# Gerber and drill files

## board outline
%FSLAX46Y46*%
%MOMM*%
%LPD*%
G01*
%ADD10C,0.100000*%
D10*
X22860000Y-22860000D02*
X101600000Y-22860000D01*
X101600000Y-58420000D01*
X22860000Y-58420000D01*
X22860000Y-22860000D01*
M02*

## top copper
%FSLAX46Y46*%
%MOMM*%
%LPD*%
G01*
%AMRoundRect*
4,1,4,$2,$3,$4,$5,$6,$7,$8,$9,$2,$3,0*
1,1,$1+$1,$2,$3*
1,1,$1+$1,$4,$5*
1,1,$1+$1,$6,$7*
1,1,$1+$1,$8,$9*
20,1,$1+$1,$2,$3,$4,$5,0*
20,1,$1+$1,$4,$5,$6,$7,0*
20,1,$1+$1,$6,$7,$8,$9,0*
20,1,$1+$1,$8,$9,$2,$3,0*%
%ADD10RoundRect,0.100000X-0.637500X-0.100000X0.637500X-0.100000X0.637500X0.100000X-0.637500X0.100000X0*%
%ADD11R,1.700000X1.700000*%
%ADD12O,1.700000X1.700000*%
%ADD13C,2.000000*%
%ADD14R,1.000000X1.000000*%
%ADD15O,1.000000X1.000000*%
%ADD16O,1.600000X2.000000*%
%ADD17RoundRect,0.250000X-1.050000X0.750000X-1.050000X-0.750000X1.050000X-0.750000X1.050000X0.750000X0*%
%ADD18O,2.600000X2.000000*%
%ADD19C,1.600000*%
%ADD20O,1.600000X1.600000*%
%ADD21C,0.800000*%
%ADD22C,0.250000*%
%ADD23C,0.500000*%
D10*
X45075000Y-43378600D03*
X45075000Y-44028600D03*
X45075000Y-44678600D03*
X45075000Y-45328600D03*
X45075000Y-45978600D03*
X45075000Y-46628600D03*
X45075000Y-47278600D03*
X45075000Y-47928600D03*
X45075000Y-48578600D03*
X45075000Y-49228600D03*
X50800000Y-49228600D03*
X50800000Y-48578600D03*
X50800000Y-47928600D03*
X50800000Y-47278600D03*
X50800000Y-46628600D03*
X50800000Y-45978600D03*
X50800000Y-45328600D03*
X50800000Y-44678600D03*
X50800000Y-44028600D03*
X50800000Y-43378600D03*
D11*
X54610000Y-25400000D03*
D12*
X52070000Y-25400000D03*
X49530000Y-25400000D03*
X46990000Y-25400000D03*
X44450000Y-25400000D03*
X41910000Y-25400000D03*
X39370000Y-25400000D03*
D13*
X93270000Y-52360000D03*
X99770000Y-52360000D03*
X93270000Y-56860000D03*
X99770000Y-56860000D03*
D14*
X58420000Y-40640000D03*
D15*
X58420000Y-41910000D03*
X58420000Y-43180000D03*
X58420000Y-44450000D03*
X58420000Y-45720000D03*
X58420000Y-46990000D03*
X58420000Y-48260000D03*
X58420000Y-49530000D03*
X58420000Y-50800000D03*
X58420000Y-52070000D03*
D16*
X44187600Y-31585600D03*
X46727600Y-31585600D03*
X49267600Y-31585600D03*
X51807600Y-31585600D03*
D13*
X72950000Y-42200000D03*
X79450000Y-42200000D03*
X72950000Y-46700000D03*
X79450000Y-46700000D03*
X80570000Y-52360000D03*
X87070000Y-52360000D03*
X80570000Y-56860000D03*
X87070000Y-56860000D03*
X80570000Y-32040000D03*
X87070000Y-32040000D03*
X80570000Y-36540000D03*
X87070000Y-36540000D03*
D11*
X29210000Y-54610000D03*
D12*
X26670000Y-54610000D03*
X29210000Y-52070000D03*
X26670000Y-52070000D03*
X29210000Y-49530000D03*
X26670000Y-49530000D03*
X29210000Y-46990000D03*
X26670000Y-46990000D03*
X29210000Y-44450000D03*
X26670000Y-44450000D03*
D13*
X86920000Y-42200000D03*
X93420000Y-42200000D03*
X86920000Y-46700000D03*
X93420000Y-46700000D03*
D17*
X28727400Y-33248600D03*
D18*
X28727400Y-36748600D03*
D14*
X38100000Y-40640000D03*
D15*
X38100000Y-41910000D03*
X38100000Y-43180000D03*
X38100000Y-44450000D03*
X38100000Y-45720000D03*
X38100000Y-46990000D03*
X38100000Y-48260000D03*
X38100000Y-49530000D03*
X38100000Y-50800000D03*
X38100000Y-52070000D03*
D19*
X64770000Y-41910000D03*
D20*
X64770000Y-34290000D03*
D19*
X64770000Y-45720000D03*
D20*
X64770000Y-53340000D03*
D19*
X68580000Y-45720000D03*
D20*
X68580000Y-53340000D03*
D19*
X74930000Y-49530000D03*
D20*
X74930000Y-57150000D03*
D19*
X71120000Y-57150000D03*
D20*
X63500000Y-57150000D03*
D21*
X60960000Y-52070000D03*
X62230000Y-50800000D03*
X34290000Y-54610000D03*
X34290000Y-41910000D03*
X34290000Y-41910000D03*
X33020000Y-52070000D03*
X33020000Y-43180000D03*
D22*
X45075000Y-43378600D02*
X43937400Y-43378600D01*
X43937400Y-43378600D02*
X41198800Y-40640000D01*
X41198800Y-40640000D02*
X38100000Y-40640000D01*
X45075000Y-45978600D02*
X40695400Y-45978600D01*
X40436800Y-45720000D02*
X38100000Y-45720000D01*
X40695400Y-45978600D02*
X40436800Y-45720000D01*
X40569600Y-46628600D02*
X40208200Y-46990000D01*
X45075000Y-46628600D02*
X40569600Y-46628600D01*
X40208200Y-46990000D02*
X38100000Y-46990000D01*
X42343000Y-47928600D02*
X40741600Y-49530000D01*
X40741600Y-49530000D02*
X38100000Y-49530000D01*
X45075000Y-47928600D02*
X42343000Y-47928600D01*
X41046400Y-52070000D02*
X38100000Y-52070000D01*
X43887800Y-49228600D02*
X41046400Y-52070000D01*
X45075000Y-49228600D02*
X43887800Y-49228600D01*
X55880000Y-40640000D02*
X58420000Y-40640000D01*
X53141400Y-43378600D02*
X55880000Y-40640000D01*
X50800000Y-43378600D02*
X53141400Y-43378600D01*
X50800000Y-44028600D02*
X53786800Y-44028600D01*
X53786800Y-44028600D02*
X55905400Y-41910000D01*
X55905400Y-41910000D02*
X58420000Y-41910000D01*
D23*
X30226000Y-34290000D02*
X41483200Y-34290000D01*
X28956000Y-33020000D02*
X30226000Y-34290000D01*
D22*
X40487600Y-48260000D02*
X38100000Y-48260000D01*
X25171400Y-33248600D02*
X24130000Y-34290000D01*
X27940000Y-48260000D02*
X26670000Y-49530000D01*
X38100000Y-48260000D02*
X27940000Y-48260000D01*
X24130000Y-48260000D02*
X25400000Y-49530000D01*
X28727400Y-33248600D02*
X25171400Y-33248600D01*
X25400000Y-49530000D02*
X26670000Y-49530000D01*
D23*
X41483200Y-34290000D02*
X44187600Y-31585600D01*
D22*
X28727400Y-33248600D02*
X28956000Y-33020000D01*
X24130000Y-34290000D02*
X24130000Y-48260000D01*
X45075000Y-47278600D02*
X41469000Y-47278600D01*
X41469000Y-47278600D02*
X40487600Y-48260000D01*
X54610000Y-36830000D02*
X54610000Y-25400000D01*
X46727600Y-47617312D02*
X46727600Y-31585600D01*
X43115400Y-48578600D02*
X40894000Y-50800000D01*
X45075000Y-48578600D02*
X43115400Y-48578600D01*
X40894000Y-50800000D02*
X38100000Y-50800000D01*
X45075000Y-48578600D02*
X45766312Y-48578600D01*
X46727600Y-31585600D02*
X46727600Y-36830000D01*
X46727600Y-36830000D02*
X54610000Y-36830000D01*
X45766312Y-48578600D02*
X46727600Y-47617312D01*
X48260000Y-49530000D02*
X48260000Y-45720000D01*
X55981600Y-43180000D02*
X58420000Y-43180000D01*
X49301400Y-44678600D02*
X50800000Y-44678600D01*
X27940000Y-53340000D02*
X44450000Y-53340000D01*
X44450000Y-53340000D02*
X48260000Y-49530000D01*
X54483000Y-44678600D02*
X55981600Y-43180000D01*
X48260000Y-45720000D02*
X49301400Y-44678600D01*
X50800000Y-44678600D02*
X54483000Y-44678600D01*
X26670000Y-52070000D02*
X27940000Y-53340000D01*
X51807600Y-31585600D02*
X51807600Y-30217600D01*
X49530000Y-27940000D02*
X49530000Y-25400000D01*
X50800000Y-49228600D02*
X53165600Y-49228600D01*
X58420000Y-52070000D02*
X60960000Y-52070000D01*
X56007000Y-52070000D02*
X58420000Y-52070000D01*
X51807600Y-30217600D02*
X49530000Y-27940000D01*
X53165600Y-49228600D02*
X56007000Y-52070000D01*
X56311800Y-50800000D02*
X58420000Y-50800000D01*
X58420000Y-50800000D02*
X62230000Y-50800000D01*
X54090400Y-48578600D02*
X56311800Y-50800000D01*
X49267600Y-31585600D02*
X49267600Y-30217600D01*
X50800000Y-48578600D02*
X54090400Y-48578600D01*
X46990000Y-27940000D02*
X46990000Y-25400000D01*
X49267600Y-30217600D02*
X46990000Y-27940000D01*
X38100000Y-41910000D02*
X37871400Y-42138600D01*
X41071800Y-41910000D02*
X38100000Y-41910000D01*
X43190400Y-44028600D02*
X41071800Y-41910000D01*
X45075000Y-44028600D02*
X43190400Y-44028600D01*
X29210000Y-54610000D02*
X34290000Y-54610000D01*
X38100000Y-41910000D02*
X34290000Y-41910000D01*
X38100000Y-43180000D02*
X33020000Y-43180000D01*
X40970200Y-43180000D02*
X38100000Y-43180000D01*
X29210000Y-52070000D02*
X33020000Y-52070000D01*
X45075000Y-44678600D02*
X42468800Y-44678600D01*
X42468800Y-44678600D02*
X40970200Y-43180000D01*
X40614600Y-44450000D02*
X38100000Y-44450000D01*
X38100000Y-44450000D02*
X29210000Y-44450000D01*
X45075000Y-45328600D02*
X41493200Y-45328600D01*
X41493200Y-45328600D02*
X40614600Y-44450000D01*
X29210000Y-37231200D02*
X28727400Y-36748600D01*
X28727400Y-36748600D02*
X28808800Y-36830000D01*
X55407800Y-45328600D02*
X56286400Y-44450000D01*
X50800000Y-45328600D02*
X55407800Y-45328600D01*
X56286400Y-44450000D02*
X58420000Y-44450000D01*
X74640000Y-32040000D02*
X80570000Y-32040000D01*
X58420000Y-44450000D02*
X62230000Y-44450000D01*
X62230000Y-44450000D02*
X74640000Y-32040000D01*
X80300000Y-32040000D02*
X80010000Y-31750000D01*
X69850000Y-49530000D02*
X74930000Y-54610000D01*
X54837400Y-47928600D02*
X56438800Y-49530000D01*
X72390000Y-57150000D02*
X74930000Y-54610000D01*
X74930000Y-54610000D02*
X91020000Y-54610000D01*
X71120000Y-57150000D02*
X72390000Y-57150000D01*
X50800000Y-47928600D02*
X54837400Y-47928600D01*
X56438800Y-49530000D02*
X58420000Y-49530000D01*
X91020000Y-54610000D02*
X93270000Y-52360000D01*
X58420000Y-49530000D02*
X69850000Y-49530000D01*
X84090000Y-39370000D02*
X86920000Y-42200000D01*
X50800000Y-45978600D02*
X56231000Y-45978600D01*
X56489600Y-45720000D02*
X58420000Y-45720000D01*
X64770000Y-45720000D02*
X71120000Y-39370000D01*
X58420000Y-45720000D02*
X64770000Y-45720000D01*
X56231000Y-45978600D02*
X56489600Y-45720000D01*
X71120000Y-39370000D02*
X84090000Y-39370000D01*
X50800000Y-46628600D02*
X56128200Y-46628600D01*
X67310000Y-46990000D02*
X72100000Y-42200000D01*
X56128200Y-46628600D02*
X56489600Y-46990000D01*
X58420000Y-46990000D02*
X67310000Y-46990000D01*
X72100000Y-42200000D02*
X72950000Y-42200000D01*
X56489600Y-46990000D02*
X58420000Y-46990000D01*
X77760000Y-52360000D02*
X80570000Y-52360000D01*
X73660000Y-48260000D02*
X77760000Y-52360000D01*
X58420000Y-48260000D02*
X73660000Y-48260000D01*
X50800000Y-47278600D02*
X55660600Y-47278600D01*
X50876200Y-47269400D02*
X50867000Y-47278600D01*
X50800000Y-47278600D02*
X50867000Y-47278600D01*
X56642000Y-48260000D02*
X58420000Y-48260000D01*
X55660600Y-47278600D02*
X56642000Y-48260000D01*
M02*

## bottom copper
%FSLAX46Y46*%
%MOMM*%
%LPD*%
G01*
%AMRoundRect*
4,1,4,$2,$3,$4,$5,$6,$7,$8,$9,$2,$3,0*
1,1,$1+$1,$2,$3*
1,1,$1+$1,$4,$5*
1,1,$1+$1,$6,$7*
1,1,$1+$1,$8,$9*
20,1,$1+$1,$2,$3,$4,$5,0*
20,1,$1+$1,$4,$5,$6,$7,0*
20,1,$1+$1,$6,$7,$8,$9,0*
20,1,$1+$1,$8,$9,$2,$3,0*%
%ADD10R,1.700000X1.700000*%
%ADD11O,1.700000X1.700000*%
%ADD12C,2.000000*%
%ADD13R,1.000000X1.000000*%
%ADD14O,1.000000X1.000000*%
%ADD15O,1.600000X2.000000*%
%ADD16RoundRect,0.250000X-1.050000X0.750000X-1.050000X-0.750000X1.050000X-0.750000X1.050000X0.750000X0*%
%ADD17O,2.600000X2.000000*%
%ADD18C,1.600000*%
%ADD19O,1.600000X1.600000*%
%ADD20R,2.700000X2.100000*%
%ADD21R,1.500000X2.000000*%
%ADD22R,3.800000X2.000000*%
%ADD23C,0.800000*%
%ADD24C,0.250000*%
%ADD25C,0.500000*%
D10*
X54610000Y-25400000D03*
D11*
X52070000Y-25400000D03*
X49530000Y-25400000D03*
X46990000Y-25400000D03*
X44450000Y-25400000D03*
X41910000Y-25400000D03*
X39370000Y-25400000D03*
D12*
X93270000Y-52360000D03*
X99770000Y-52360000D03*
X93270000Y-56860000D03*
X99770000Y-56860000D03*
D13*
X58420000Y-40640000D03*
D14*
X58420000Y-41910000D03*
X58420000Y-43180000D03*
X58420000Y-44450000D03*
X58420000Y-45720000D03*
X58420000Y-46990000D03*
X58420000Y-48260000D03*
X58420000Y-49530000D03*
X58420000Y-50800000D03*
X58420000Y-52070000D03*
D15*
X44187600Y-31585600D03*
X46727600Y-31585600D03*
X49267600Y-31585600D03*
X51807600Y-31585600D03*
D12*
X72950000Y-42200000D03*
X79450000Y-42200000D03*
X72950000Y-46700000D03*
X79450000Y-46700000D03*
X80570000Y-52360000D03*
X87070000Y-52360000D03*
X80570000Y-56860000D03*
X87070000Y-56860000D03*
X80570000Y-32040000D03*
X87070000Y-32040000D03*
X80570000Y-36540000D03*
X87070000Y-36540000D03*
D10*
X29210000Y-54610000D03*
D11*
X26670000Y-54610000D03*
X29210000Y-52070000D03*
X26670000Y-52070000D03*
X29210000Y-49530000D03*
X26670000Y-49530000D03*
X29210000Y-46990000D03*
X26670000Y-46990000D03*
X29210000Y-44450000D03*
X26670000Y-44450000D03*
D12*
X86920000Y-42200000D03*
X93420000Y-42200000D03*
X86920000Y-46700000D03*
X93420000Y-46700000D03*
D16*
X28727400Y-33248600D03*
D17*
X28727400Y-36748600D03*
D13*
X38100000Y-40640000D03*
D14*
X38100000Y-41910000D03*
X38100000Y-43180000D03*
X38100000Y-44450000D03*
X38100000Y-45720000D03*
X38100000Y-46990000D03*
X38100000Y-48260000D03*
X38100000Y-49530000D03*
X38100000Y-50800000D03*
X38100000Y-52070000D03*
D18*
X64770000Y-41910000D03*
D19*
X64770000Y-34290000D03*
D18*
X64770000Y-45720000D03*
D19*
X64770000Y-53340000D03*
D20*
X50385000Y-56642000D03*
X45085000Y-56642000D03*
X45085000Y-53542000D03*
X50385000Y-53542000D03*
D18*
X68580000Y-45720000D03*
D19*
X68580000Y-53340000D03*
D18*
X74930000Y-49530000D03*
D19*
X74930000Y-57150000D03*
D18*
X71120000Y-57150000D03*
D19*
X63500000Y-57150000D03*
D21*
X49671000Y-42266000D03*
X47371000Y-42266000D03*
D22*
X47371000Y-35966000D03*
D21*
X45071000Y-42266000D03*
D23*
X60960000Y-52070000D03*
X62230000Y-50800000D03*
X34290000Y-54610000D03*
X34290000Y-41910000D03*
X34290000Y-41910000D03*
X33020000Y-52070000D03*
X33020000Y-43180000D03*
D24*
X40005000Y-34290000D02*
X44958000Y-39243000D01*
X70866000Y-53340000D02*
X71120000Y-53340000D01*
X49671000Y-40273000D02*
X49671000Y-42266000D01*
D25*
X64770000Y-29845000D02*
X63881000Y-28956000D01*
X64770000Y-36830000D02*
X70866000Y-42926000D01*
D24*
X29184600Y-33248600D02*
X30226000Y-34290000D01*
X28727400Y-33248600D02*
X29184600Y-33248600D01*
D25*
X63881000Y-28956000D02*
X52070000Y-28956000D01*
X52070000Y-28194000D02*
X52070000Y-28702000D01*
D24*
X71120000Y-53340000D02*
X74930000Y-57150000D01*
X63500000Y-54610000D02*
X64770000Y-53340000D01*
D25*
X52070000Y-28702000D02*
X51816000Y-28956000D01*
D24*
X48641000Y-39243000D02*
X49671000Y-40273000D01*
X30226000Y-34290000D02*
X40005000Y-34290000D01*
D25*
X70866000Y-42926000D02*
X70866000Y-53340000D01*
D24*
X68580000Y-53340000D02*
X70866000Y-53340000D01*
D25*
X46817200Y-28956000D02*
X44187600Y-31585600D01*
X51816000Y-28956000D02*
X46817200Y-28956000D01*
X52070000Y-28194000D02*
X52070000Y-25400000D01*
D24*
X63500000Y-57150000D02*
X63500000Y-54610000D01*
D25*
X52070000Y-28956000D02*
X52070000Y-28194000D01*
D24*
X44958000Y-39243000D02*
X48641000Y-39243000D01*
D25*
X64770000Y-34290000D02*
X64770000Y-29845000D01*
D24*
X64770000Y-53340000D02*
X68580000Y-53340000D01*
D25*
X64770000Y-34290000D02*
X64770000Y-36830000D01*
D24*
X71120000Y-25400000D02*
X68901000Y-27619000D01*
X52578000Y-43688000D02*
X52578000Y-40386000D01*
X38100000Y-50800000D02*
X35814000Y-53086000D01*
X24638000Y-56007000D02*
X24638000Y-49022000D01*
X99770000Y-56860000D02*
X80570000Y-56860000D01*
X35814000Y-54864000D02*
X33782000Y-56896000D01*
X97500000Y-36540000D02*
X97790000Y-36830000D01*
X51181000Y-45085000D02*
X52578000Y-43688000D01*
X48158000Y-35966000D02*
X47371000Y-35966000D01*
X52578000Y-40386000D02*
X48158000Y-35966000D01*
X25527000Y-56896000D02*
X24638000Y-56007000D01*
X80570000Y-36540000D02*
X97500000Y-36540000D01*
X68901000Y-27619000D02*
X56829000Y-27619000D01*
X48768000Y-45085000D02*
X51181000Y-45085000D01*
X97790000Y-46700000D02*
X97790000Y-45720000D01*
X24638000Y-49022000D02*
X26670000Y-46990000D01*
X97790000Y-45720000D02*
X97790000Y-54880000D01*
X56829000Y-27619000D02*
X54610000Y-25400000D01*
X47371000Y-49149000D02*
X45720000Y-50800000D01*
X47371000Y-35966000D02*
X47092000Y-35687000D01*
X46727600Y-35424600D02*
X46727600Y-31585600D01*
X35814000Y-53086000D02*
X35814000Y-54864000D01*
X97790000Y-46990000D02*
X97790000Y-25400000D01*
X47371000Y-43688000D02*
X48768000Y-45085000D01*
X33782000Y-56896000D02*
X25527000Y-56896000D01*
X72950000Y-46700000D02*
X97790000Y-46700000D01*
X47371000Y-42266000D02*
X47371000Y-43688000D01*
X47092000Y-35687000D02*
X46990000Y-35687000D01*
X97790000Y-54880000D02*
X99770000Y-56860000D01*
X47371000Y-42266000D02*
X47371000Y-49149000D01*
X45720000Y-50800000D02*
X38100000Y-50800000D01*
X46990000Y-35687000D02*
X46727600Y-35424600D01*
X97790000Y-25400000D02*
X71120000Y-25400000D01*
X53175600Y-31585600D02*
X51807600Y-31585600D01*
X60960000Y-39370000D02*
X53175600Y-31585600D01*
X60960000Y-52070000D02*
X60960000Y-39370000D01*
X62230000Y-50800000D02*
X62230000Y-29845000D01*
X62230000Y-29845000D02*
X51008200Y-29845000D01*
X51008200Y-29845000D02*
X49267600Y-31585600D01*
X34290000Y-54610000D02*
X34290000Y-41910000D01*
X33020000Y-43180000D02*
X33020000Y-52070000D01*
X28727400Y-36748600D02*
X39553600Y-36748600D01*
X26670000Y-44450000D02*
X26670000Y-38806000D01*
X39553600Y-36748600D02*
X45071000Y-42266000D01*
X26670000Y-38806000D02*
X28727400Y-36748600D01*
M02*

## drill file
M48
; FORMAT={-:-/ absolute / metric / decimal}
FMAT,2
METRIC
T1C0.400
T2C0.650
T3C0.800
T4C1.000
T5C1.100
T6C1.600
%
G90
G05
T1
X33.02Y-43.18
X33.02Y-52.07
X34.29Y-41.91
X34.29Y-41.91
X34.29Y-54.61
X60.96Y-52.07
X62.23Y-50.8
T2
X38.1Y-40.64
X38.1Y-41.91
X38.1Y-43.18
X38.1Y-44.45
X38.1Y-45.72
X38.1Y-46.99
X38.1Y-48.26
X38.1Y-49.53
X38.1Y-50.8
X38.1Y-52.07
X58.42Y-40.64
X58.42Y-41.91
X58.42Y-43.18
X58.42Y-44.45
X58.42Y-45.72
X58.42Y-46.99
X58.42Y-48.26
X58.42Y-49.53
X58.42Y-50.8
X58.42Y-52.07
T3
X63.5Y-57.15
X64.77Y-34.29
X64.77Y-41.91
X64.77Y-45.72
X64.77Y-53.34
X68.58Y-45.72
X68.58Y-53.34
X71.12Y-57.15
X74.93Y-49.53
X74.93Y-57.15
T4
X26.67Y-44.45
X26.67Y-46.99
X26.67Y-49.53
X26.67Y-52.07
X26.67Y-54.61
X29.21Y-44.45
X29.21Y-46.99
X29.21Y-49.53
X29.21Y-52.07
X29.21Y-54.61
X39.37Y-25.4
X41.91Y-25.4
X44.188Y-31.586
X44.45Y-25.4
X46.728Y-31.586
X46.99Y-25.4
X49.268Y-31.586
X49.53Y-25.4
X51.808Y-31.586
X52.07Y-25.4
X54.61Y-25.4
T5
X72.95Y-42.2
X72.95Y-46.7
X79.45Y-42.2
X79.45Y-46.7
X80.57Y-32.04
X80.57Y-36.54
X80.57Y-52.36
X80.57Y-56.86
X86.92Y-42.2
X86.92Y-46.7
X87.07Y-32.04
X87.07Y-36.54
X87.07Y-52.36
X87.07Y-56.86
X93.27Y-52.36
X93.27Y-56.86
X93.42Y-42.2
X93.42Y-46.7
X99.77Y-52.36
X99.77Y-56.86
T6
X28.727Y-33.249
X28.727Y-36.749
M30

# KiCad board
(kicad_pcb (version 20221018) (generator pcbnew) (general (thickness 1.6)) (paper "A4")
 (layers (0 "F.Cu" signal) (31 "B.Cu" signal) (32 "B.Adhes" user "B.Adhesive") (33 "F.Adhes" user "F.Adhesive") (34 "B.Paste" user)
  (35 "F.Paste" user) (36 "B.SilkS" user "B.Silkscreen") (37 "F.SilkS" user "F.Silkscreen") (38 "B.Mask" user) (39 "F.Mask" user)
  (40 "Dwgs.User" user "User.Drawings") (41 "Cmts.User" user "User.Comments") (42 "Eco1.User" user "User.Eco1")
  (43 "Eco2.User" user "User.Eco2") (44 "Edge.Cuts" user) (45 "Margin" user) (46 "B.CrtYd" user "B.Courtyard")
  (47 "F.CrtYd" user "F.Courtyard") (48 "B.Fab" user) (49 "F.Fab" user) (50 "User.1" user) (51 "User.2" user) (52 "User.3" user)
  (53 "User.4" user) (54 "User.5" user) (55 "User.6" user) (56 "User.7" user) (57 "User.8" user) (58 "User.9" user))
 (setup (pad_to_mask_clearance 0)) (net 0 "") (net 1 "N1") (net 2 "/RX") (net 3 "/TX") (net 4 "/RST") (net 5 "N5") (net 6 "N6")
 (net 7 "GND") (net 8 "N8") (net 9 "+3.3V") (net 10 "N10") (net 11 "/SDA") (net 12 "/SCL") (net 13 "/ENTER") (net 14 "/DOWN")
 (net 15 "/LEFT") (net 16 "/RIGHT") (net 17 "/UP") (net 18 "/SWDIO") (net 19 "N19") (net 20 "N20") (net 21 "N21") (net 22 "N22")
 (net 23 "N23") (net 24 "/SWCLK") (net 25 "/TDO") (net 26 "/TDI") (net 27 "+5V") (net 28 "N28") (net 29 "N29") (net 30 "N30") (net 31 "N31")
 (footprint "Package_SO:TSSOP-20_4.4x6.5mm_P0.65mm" (layer "F.Cu") (at 47.9375 46.3036)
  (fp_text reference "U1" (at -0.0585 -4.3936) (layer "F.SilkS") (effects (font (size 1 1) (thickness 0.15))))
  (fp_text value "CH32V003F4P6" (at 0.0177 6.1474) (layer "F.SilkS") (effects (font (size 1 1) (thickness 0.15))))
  (pad "1" smd roundrect (at -2.8625 -2.925) (size 1.475 0.4) (layers "F.Cu" "F.Paste" "F.Mask") (roundrect_rratio 0.25) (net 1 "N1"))
  (pad "2" smd roundrect (at -2.8625 -2.275) (size 1.475 0.4) (layers "F.Cu" "F.Paste" "F.Mask") (roundrect_rratio 0.25) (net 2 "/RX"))
  (pad "3" smd roundrect (at -2.8625 -1.625) (size 1.475 0.4) (layers "F.Cu" "F.Paste" "F.Mask") (roundrect_rratio 0.25) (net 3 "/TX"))
  (pad "4" smd roundrect (at -2.8625 -0.975) (size 1.475 0.4) (layers "F.Cu" "F.Paste" "F.Mask") (roundrect_rratio 0.25) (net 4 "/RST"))
  (pad "5" smd roundrect (at -2.8625 -0.325) (size 1.475 0.4) (layers "F.Cu" "F.Paste" "F.Mask") (roundrect_rratio 0.25) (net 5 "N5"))
  (pad "6" smd roundrect (at -2.8625 0.325) (size 1.475 0.4) (layers "F.Cu" "F.Paste" "F.Mask") (roundrect_rratio 0.25) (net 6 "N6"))
  (pad "7" smd roundrect (at -2.8625 0.975) (size 1.475 0.4) (layers "F.Cu" "F.Paste" "F.Mask") (roundrect_rratio 0.25) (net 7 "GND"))
  (pad "8" smd roundrect (at -2.8625 1.625) (size 1.475 0.4) (layers "F.Cu" "F.Paste" "F.Mask") (roundrect_rratio 0.25) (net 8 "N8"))
  (pad "9" smd roundrect (at -2.8625 2.275) (size 1.475 0.4) (layers "F.Cu" "F.Paste" "F.Mask") (roundrect_rratio 0.25) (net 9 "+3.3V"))
  (pad "10" smd roundrect (at -2.8625 2.925) (size 1.475 0.4) (layers "F.Cu" "F.Paste" "F.Mask") (roundrect_rratio 0.25) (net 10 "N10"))
  (pad "11" smd roundrect (at 2.8625 2.925) (size 1.475 0.4) (layers "F.Cu" "F.Paste" "F.Mask") (roundrect_rratio 0.25) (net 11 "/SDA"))
  (pad "12" smd roundrect (at 2.8625 2.275) (size 1.475 0.4) (layers "F.Cu" "F.Paste" "F.Mask") (roundrect_rratio 0.25) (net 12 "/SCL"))
  (pad "13" smd roundrect (at 2.8625 1.625) (size 1.475 0.4) (layers "F.Cu" "F.Paste" "F.Mask") (roundrect_rratio 0.25) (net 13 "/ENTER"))
  (pad "14" smd roundrect (at 2.8625 0.975) (size 1.475 0.4) (layers "F.Cu" "F.Paste" "F.Mask") (roundrect_rratio 0.25) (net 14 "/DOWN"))
  (pad "15" smd roundrect (at 2.8625 0.325) (size 1.475 0.4) (layers "F.Cu" "F.Paste" "F.Mask") (roundrect_rratio 0.25) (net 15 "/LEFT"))
  (pad "16" smd roundrect (at 2.8625 -0.325) (size 1.475 0.4) (layers "F.Cu" "F.Paste" "F.Mask") (roundrect_rratio 0.25) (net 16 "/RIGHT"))
  (pad "17" smd roundrect (at 2.8625 -0.975) (size 1.475 0.4) (layers "F.Cu" "F.Paste" "F.Mask") (roundrect_rratio 0.25) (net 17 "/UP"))
  (pad "18" smd roundrect (at 2.8625 -1.625) (size 1.475 0.4) (layers "F.Cu" "F.Paste" "F.Mask") (roundrect_rratio 0.25) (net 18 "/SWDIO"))
  (pad "19" smd roundrect (at 2.8625 -2.275) (size 1.475 0.4) (layers "F.Cu" "F.Paste" "F.Mask") (roundrect_rratio 0.25) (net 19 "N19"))
  (pad "20" smd roundrect (at 2.8625 -2.925) (size 1.475 0.4) (layers "F.Cu" "F.Paste" "F.Mask") (roundrect_rratio 0.25) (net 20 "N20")))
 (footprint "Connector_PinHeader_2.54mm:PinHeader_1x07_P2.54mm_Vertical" (layer "F.Cu") (at 54.61 25.4 -90)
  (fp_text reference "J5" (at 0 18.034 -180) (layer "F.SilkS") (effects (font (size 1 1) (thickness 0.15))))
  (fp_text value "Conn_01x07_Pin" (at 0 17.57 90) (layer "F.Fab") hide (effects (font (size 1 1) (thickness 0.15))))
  (pad "1" thru_hole rect (at 0 0 270) (size 1.7 1.7) (drill 1) (layers "*.Cu" "*.Mask") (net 9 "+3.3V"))
  (pad "2" thru_hole oval (at 0 2.54 270) (size 1.7 1.7) (drill 1) (layers "*.Cu" "*.Mask") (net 7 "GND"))
  (pad "3" thru_hole oval (at 0 5.08 270) (size 1.7 1.7) (drill 1) (layers "*.Cu" "*.Mask") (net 11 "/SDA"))
  (pad "4" thru_hole oval (at 0 7.62 270) (size 1.7 1.7) (drill 1) (layers "*.Cu" "*.Mask") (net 12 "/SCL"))
  (pad "5" thru_hole oval (at 0 10.16 270) (size 1.7 1.7) (drill 1) (layers "*.Cu" "*.Mask") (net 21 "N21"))
  (pad "6" thru_hole oval (at 0 12.7 270) (size 1.7 1.7) (drill 1) (layers "*.Cu" "*.Mask") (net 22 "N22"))
  (pad "7" thru_hole oval (at 0 15.24 270) (size 1.7 1.7) (drill 1) (layers "*.Cu" "*.Mask") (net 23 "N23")))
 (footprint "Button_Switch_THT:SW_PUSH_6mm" (layer "F.Cu") (at 93.27 52.36)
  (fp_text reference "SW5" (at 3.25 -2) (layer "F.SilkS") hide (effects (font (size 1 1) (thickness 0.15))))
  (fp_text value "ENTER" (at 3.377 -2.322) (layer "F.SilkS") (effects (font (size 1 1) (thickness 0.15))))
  (pad "1" thru_hole circle (at 0 0 90) (size 2 2) (drill 1.1) (layers "*.Cu" "*.Mask") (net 13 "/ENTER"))
  (pad "1" thru_hole circle (at 6.5 0 90) (size 2 2) (drill 1.1) (layers "*.Cu" "*.Mask") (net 13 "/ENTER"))
  (pad "2" thru_hole circle (at 0 4.5 90) (size 2 2) (drill 1.1) (layers "*.Cu" "*.Mask") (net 9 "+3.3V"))
  (pad "2" thru_hole circle (at 6.5 4.5 90) (size 2 2) (drill 1.1) (layers "*.Cu" "*.Mask") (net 9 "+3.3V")))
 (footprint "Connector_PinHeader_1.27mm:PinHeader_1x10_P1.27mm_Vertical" (layer "F.Cu") (at 58.42 40.64)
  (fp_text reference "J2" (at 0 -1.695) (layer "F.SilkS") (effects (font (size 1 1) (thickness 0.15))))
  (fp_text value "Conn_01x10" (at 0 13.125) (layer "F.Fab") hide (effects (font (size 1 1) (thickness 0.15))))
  (pad "1" thru_hole rect (at 0 0) (size 1 1) (drill 0.65) (layers "*.Cu" "*.Mask") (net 20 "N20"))
  (pad "2" thru_hole oval (at 0 1.27) (size 1 1) (drill 0.65) (layers "*.Cu" "*.Mask") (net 19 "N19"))
  (pad "3" thru_hole oval (at 0 2.54) (size 1 1) (drill 0.65) (layers "*.Cu" "*.Mask") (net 18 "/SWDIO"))
  (pad "4" thru_hole oval (at 0 3.81) (size 1 1) (drill 0.65) (layers "*.Cu" "*.Mask") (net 17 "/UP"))
  (pad "5" thru_hole oval (at 0 5.08) (size 1 1) (drill 0.65) (layers "*.Cu" "*.Mask") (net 16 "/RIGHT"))
  (pad "6" thru_hole oval (at 0 6.35) (size 1 1) (drill 0.65) (layers "*.Cu" "*.Mask") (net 15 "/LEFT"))
  (pad "7" thru_hole oval (at 0 7.62) (size 1 1) (drill 0.65) (layers "*.Cu" "*.Mask") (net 14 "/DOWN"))
  (pad "8" thru_hole oval (at 0 8.89) (size 1 1) (drill 0.65) (layers "*.Cu" "*.Mask") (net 13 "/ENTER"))
  (pad "9" thru_hole oval (at 0 10.16) (size 1 1) (drill 0.65) (layers "*.Cu" "*.Mask") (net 12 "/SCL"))
  (pad "10" thru_hole oval (at 0 11.43) (size 1 1) (drill 0.65) (layers "*.Cu" "*.Mask") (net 11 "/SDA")))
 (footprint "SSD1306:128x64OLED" (layer "F.Cu") (at 47.8076 42.1856)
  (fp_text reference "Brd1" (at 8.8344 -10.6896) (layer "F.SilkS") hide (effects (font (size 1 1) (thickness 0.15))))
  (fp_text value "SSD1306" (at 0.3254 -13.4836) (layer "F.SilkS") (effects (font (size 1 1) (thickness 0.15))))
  (pad "1" thru_hole oval (at -3.62 -10.6 90) (size 2 1.6) (drill 1) (layers "*.Cu" "*.Mask") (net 7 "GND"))
  (pad "2" thru_hole oval (at -1.08 -10.6 90) (size 2 1.6) (drill 1) (layers "*.Cu" "*.Mask") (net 9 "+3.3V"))
  (pad "3" thru_hole oval (at 1.46 -10.6 90) (size 2 1.6) (drill 1) (layers "*.Cu" "*.Mask") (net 12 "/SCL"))
  (pad "4" thru_hole oval (at 4 -10.6 90) (size 2 1.6) (drill 1) (layers "*.Cu" "*.Mask") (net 11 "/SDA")))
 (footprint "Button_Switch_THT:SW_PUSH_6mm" (layer "F.Cu") (at 72.95 42.2)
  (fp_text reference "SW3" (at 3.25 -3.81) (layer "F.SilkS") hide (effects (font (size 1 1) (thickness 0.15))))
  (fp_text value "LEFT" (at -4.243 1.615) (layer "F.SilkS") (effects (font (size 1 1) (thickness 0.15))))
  (pad "1" thru_hole circle (at 0 0 90) (size 2 2) (drill 1.1) (layers "*.Cu" "*.Mask") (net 15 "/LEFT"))
  (pad "1" thru_hole circle (at 6.5 0 90) (size 2 2) (drill 1.1) (layers "*.Cu" "*.Mask") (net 15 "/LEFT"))
  (pad "2" thru_hole circle (at 0 4.5 90) (size 2 2) (drill 1.1) (layers "*.Cu" "*.Mask") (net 9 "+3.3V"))
  (pad "2" thru_hole circle (at 6.5 4.5 90) (size 2 2) (drill 1.1) (layers "*.Cu" "*.Mask") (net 9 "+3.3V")))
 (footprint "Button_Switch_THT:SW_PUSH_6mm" (layer "F.Cu") (at 80.57 52.36)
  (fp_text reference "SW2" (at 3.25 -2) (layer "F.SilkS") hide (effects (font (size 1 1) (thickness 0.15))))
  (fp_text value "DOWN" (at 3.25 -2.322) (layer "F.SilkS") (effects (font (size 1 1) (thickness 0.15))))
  (pad "1" thru_hole circle (at 0 0 90) (size 2 2) (drill 1.1) (layers "*.Cu" "*.Mask") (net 14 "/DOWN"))
  (pad "1" thru_hole circle (at 6.5 0 90) (size 2 2) (drill 1.1) (layers "*.Cu" "*.Mask") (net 14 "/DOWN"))
  (pad "2" thru_hole circle (at 0 4.5 90) (size 2 2) (drill 1.1) (layers "*.Cu" "*.Mask") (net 9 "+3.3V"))
  (pad "2" thru_hole circle (at 6.5 4.5 90) (size 2 2) (drill 1.1) (layers "*.Cu" "*.Mask") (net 9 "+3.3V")))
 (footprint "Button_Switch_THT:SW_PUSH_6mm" (layer "F.Cu") (at 80.57 32.04)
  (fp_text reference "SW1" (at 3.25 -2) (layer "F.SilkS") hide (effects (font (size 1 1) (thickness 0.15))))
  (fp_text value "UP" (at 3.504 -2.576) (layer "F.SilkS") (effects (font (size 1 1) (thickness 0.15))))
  (pad "1" thru_hole circle (at 0 0 90) (size 2 2) (drill 1.1) (layers "*.Cu" "*.Mask") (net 17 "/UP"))
  (pad "1" thru_hole circle (at 6.5 0 90) (size 2 2) (drill 1.1) (layers "*.Cu" "*.Mask") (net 17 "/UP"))
  (pad "2" thru_hole circle (at 0 4.5 90) (size 2 2) (drill 1.1) (layers "*.Cu" "*.Mask") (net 9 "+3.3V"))
  (pad "2" thru_hole circle (at 6.5 4.5 90) (size 2 2) (drill 1.1) (layers "*.Cu" "*.Mask") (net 9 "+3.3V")))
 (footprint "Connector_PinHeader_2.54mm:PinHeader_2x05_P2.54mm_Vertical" (layer "F.Cu") (at 29.21 54.61 180)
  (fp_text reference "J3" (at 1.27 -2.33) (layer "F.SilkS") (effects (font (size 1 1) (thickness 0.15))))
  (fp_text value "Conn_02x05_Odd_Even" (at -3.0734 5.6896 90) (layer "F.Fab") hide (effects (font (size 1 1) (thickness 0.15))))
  (pad "1" thru_hole rect (at 0 0 180) (size 1.7 1.7) (drill 1) (layers "*.Cu" "*.Mask") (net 2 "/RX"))
  (pad "2" thru_hole oval (at 2.54 0 180) (size 1.7 1.7) (drill 1) (layers "*.Cu" "*.Mask") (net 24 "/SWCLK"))
  (pad "3" thru_hole oval (at 0 2.54 180) (size 1.7 1.7) (drill 1) (layers "*.Cu" "*.Mask") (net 3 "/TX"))
  (pad "4" thru_hole oval (at 2.54 2.54 180) (size 1.7 1.7) (drill 1) (layers "*.Cu" "*.Mask") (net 18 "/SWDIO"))
  (pad "5" thru_hole oval (at 0 5.08 180) (size 1.7 1.7) (drill 1) (layers "*.Cu" "*.Mask") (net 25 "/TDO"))
  (pad "6" thru_hole oval (at 2.54 5.08 180) (size 1.7 1.7) (drill 1) (layers "*.Cu" "*.Mask") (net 7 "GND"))
  (pad "7" thru_hole oval (at 0 7.62 180) (size 1.7 1.7) (drill 1) (layers "*.Cu" "*.Mask") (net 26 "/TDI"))
  (pad "8" thru_hole oval (at 2.54 7.62 180) (size 1.7 1.7) (drill 1) (layers "*.Cu" "*.Mask") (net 9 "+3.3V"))
  (pad "9" thru_hole oval (at 0 10.16 180) (size 1.7 1.7) (drill 1) (layers "*.Cu" "*.Mask") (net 4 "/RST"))
  (pad "10" thru_hole oval (at 2.54 10.16 180) (size 1.7 1.7) (drill 1) (layers "*.Cu" "*.Mask") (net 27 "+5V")))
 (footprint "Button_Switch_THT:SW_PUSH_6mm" (layer "F.Cu") (at 86.92 42.2)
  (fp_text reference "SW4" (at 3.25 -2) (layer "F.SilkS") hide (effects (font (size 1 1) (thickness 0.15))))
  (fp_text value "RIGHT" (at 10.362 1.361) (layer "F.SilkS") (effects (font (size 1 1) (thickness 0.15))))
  (pad "1" thru_hole circle (at 0 0 90) (size 2 2) (drill 1.1) (layers "*.Cu" "*.Mask") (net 16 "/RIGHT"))
  (pad "1" thru_hole circle (at 6.5 0 90) (size 2 2) (drill 1.1) (layers "*.Cu" "*.Mask") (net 16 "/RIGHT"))
  (pad "2" thru_hole circle (at 0 4.5 90) (size 2 2) (drill 1.1) (layers "*.Cu" "*.Mask") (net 9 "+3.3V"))
  (pad "2" thru_hole circle (at 6.5 4.5 90) (size 2 2) (drill 1.1) (layers "*.Cu" "*.Mask") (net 9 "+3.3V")))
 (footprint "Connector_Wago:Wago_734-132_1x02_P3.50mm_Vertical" (layer "F.Cu") (at 28.7274 33.2486 -90)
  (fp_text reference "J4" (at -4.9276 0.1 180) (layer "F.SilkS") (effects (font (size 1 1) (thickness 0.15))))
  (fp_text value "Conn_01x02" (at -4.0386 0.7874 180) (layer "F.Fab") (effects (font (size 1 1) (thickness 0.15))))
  (pad "1" thru_hole roundrect (at 0 0 270) (size 2 2.6) (drill 1.6) (layers "*.Cu" "*.Mask") (roundrect_rratio 0.125) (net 7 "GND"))
  (pad "2" thru_hole oval (at 3.5 0 270) (size 2 2.6) (drill 1.6) (layers "*.Cu" "*.Mask") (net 27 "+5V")))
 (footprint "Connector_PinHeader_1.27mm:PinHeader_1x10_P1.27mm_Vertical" (layer "F.Cu") (at 38.1 40.64)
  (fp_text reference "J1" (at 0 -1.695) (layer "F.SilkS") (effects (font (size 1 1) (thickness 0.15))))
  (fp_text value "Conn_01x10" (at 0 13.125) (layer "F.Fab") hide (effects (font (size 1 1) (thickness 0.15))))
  (pad "1" thru_hole rect (at 0 0) (size 1 1) (drill 0.65) (layers "*.Cu" "*.Mask") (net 1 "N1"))
  (pad "2" thru_hole oval (at 0 1.27) (size 1 1) (drill 0.65) (layers "*.Cu" "*.Mask") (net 2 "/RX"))
  (pad "3" thru_hole oval (at 0 2.54) (size 1 1) (drill 0.65) (layers "*.Cu" "*.Mask") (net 3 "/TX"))
  (pad "4" thru_hole oval (at 0 3.81) (size 1 1) (drill 0.65) (layers "*.Cu" "*.Mask") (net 4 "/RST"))
  (pad "5" thru_hole oval (at 0 5.08) (size 1 1) (drill 0.65) (layers "*.Cu" "*.Mask") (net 5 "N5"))
  (pad "6" thru_hole oval (at 0 6.35) (size 1 1) (drill 0.65) (layers "*.Cu" "*.Mask") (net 6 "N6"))
  (pad "7" thru_hole oval (at 0 7.62) (size 1 1) (drill 0.65) (layers "*.Cu" "*.Mask") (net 7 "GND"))
  (pad "8" thru_hole oval (at 0 8.89) (size 1 1) (drill 0.65) (layers "*.Cu" "*.Mask") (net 8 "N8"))
  (pad "9" thru_hole oval (at 0 10.16) (size 1 1) (drill 0.65) (layers "*.Cu" "*.Mask") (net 9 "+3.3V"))
  (pad "10" thru_hole oval (at 0 11.43) (size 1 1) (drill 0.65) (layers "*.Cu" "*.Mask") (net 10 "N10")))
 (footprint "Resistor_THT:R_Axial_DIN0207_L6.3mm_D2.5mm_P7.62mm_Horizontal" (layer "B.Cu") (at 64.77 41.91 90)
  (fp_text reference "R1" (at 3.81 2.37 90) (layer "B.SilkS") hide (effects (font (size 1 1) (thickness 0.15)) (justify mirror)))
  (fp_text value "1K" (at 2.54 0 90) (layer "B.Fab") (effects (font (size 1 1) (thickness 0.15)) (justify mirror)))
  (pad "1" thru_hole circle (at 0 0 90) (size 1.6 1.6) (drill 0.8) (layers "*.Cu" "*.Mask") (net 17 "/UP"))
  (pad "2" thru_hole oval (at 7.62 0 90) (size 1.6 1.6) (drill 0.8) (layers "*.Cu" "*.Mask") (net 7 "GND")))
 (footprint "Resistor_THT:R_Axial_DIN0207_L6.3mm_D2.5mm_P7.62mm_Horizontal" (layer "B.Cu") (at 64.77 45.72 -90)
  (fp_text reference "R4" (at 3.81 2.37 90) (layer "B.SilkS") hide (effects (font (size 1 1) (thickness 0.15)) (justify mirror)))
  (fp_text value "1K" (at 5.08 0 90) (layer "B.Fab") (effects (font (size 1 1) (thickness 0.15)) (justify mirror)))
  (pad "1" thru_hole circle (at 0 0 270) (size 1.6 1.6) (drill 0.8) (layers "*.Cu" "*.Mask") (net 16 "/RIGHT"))
  (pad "2" thru_hole oval (at 7.62 0 270) (size 1.6 1.6) (drill 0.8) (layers "*.Cu" "*.Mask") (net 7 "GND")))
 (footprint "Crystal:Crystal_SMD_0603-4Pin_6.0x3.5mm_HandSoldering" (layer "B.Cu") (at 47.735 55.092 180)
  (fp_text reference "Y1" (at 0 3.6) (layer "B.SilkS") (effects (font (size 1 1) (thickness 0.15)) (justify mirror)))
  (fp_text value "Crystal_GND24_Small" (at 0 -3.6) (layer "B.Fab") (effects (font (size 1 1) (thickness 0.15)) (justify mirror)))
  (pad "1" smd rect (at -2.65 -1.55 180) (size 2.7 2.1) (layers "B.Cu" "B.Paste" "B.Mask") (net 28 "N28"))
  (pad "2" smd rect (at 2.65 -1.55 180) (size 2.7 2.1) (layers "B.Cu" "B.Paste" "B.Mask") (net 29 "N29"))
  (pad "3" smd rect (at 2.65 1.55 180) (size 2.7 2.1) (layers "B.Cu" "B.Paste" "B.Mask") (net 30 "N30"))
  (pad "4" smd rect (at -2.65 1.55 180) (size 2.7 2.1) (layers "B.Cu" "B.Paste" "B.Mask") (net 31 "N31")))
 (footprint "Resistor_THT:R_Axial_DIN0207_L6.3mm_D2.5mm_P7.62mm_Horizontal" (layer "B.Cu") (at 68.58 45.72 -90)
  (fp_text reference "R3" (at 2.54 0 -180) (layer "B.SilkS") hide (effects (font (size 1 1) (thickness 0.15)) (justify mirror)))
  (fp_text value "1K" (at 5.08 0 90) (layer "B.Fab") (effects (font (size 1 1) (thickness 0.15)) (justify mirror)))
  (pad "1" thru_hole circle (at 0 0 270) (size 1.6 1.6) (drill 0.8) (layers "*.Cu" "*.Mask") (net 15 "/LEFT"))
  (pad "2" thru_hole oval (at 7.62 0 270) (size 1.6 1.6) (drill 0.8) (layers "*.Cu" "*.Mask") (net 7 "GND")))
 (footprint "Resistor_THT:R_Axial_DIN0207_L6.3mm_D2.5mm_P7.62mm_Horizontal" (layer "B.Cu") (at 74.93 49.53 -90)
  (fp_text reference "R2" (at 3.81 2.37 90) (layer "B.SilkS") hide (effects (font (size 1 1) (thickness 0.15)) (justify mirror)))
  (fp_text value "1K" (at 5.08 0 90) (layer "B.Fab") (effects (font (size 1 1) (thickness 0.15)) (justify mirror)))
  (pad "1" thru_hole circle (at 0 0 270) (size 1.6 1.6) (drill 0.8) (layers "*.Cu" "*.Mask") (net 14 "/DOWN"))
  (pad "2" thru_hole oval (at 7.62 0 270) (size 1.6 1.6) (drill 0.8) (layers "*.Cu" "*.Mask") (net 7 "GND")))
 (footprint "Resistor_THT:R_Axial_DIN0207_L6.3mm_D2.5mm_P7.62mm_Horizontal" (layer "B.Cu") (at 71.12 57.15 180)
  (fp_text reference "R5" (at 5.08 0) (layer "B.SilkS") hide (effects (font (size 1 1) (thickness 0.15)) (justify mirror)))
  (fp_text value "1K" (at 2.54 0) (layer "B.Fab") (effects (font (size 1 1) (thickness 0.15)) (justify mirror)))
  (pad "1" thru_hole circle (at 0 0 180) (size 1.6 1.6) (drill 0.8) (layers "*.Cu" "*.Mask") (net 13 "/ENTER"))
  (pad "2" thru_hole oval (at 7.62 0 180) (size 1.6 1.6) (drill 0.8) (layers "*.Cu" "*.Mask") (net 7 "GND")))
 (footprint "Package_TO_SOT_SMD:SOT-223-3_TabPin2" (layer "B.Cu") (at 47.371 39.116 90)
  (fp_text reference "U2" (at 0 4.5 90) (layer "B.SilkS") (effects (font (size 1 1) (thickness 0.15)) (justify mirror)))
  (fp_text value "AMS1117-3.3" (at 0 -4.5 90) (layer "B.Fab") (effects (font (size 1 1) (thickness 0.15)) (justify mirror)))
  (pad "1" smd rect (at -3.15 2.3 90) (size 2 1.5) (layers "B.Cu" "B.Paste" "B.Mask") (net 7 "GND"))
  (pad "2" smd rect (at -3.15 0 90) (size 2 1.5) (layers "B.Cu" "B.Paste" "B.Mask") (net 9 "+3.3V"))
  (pad "2" smd rect (at 3.15 0 90) (size 2 3.8) (layers "B.Cu" "B.Paste" "B.Mask") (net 9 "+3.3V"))
  (pad "3" smd rect (at -3.15 -2.3 90) (size 2 1.5) (layers "B.Cu" "B.Paste" "B.Mask") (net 27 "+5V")))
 (gr_rect (start 22.86 22.86) (end 101.6 58.42) (stroke (width 0.1) (type default)) (fill none) (layer "Edge.Cuts"))
 (segment (start 45.075 43.3786) (end 43.9374 43.3786) (width 0.25) (layer "F.Cu") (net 1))
 (segment (start 43.9374 43.3786) (end 41.1988 40.64) (width 0.25) (layer "F.Cu") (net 1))
 (segment (start 41.1988 40.64) (end 38.1 40.64) (width 0.25) (layer "F.Cu") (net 1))
 (segment (start 45.075 45.9786) (end 40.6954 45.9786) (width 0.25) (layer "F.Cu") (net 5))
 (segment (start 40.4368 45.72) (end 38.1 45.72) (width 0.25) (layer "F.Cu") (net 5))
 (segment (start 40.6954 45.9786) (end 40.4368 45.72) (width 0.25) (layer "F.Cu") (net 5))
 (segment (start 40.5696 46.6286) (end 40.2082 46.99) (width 0.25) (layer "F.Cu") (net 6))
 (segment (start 45.075 46.6286) (end 40.5696 46.6286) (width 0.25) (layer "F.Cu") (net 6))
 (segment (start 40.2082 46.99) (end 38.1 46.99) (width 0.25) (layer "F.Cu") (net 6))
 (segment (start 42.343 47.9286) (end 40.7416 49.53) (width 0.25) (layer "F.Cu") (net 8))
 (segment (start 40.7416 49.53) (end 38.1 49.53) (width 0.25) (layer "F.Cu") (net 8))
 (segment (start 45.075 47.9286) (end 42.343 47.9286) (width 0.25) (layer "F.Cu") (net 8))
 (segment (start 41.0464 52.07) (end 38.1 52.07) (width 0.25) (layer "F.Cu") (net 10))
 (segment (start 43.8878 49.2286) (end 41.0464 52.07) (width 0.25) (layer "F.Cu") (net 10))
 (segment (start 45.075 49.2286) (end 43.8878 49.2286) (width 0.25) (layer "F.Cu") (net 10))
 (segment (start 55.88 40.64) (end 58.42 40.64) (width 0.25) (layer "F.Cu") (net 20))
 (segment (start 53.1414 43.3786) (end 55.88 40.64) (width 0.25) (layer "F.Cu") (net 20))
 (segment (start 50.8 43.3786) (end 53.1414 43.3786) (width 0.25) (layer "F.Cu") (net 20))
 (segment (start 50.8 44.0286) (end 53.7868 44.0286) (width 0.25) (layer "F.Cu") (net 19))
 (segment (start 53.7868 44.0286) (end 55.9054 41.91) (width 0.25) (layer "F.Cu") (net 19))
 (segment (start 55.9054 41.91) (end 58.42 41.91) (width 0.25) (layer "F.Cu") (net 19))
 (segment (start 30.226 34.29) (end 41.4832 34.29) (width 0.5) (layer "F.Cu") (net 7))
 (segment (start 28.956 33.02) (end 30.226 34.29) (width 0.5) (layer "F.Cu") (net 7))
 (segment (start 40.4876 48.26) (end 38.1 48.26) (width 0.25) (layer "F.Cu") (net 7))
 (segment (start 25.1714 33.2486) (end 24.13 34.29) (width 0.25) (layer "F.Cu") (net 7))
 (segment (start 27.94 48.26) (end 26.67 49.53) (width 0.25) (layer "F.Cu") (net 7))
 (segment (start 38.1 48.26) (end 27.94 48.26) (width 0.25) (layer "F.Cu") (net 7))
 (segment (start 24.13 48.26) (end 25.4 49.53) (width 0.25) (layer "F.Cu") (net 7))
 (segment (start 28.7274 33.2486) (end 25.1714 33.2486) (width 0.25) (layer "F.Cu") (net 7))
 (segment (start 25.4 49.53) (end 26.67 49.53) (width 0.25) (layer "F.Cu") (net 7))
 (segment (start 41.4832 34.29) (end 44.1876 31.5856) (width 0.5) (layer "F.Cu") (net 7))
 (segment (start 28.7274 33.2486) (end 28.956 33.02) (width 0.25) (layer "F.Cu") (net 7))
 (segment (start 24.13 34.29) (end 24.13 48.26) (width 0.25) (layer "F.Cu") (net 7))
 (segment (start 45.075 47.2786) (end 41.469 47.2786) (width 0.25) (layer "F.Cu") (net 7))
 (segment (start 41.469 47.2786) (end 40.4876 48.26) (width 0.25) (layer "F.Cu") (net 7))
 (segment (start 40.005 34.29) (end 44.958 39.243) (width 0.25) (layer "B.Cu") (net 7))
 (segment (start 70.866 53.34) (end 71.12 53.34) (width 0.25) (layer "B.Cu") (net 7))
 (segment (start 49.671 40.273) (end 49.671 42.266) (width 0.25) (layer "B.Cu") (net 7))
 (segment (start 64.77 29.845) (end 63.881 28.956) (width 0.5) (layer "B.Cu") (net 7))
 (segment (start 64.77 36.83) (end 70.866 42.926) (width 0.5) (layer "B.Cu") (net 7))
 (segment (start 29.1846 33.2486) (end 30.226 34.29) (width 0.25) (layer "B.Cu") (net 7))
 (segment (start 28.7274 33.2486) (end 29.1846 33.2486) (width 0.25) (layer "B.Cu") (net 7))
 (segment (start 63.881 28.956) (end 52.07 28.956) (width 0.5) (layer "B.Cu") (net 7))
 (segment (start 52.07 28.194) (end 52.07 28.702) (width 0.5) (layer "B.Cu") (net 7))
 (segment (start 71.12 53.34) (end 74.93 57.15) (width 0.25) (layer "B.Cu") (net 7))
 (segment (start 63.5 54.61) (end 64.77 53.34) (width 0.25) (layer "B.Cu") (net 7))
 (segment (start 52.07 28.702) (end 51.816 28.956) (width 0.5) (layer "B.Cu") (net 7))
 (segment (start 48.641 39.243) (end 49.671 40.273) (width 0.25) (layer "B.Cu") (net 7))
 (segment (start 30.226 34.29) (end 40.005 34.29) (width 0.25) (layer "B.Cu") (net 7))
 (segment (start 70.866 42.926) (end 70.866 53.34) (width 0.5) (layer "B.Cu") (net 7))
 (segment (start 68.58 53.34) (end 70.866 53.34) (width 0.25) (layer "B.Cu") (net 7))
 (segment (start 46.8172 28.956) (end 44.1876 31.5856) (width 0.5) (layer "B.Cu") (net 7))
 (segment (start 51.816 28.956) (end 46.8172 28.956) (width 0.5) (layer "B.Cu") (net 7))
 (segment (start 52.07 28.194) (end 52.07 25.4) (width 0.5) (layer "B.Cu") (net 7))
 (segment (start 63.5 57.15) (end 63.5 54.61) (width 0.25) (layer "B.Cu") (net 7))
 (segment (start 52.07 28.956) (end 52.07 28.194) (width 0.5) (layer "B.Cu") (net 7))
 (segment (start 44.958 39.243) (end 48.641 39.243) (width 0.25) (layer "B.Cu") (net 7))
 (segment (start 64.77 34.29) (end 64.77 29.845) (width 0.5) (layer "B.Cu") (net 7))
 (segment (start 64.77 53.34) (end 68.58 53.34) (width 0.25) (layer "B.Cu") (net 7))
 (segment (start 64.77 34.29) (end 64.77 36.83) (width 0.5) (layer "B.Cu") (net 7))
 (segment (start 54.61 36.83) (end 54.61 25.4) (width 0.25) (layer "F.Cu") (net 9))
 (segment (start 46.7276 47.617312) (end 46.7276 31.5856) (width 0.25) (layer "F.Cu") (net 9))
 (segment (start 43.1154 48.5786) (end 40.894 50.8) (width 0.25) (layer "F.Cu") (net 9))
 (segment (start 45.075 48.5786) (end 43.1154 48.5786) (width 0.25) (layer "F.Cu") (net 9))
 (segment (start 40.894 50.8) (end 38.1 50.8) (width 0.25) (layer "F.Cu") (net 9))
 (segment (start 45.075 48.5786) (end 45.766312 48.5786) (width 0.25) (layer "F.Cu") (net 9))
 (segment (start 46.7276 31.5856) (end 46.7276 36.83) (width 0.25) (layer "F.Cu") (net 9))
 (segment (start 46.7276 36.83) (end 54.61 36.83) (width 0.25) (layer "F.Cu") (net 9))
 (segment (start 45.766312 48.5786) (end 46.7276 47.617312) (width 0.25) (layer "F.Cu") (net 9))
 (segment (start 71.12 25.4) (end 68.901 27.619) (width 0.25) (layer "B.Cu") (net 9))
 (segment (start 52.578 43.688) (end 52.578 40.386) (width 0.25) (layer "B.Cu") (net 9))
 (segment (start 38.1 50.8) (end 35.814 53.086) (width 0.25) (layer "B.Cu") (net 9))
 (segment (start 24.638 56.007) (end 24.638 49.022) (width 0.25) (layer "B.Cu") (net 9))
 (segment (start 99.77 56.86) (end 80.57 56.86) (width 0.25) (layer "B.Cu") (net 9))
 (segment (start 35.814 54.864) (end 33.782 56.896) (width 0.25) (layer "B.Cu") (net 9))
 (segment (start 97.5 36.54) (end 97.79 36.83) (width 0.25) (layer "B.Cu") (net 9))
 (segment (start 51.181 45.085) (end 52.578 43.688) (width 0.25) (layer "B.Cu") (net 9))
 (segment (start 48.158 35.966) (end 47.371 35.966) (width 0.25) (layer "B.Cu") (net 9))
 (segment (start 52.578 40.386) (end 48.158 35.966) (width 0.25) (layer "B.Cu") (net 9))
 (segment (start 25.527 56.896) (end 24.638 56.007) (width 0.25) (layer "B.Cu") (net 9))
 (segment (start 80.57 36.54) (end 97.5 36.54) (width 0.25) (layer "B.Cu") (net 9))
 (segment (start 68.901 27.619) (end 56.829 27.619) (width 0.25) (layer "B.Cu") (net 9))
 (segment (start 48.768 45.085) (end 51.181 45.085) (width 0.25) (layer "B.Cu") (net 9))
 (segment (start 97.79 46.7) (end 97.79 45.72) (width 0.25) (layer "B.Cu") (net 9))
 (segment (start 24.638 49.022) (end 26.67 46.99) (width 0.25) (layer "B.Cu") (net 9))
 (segment (start 97.79 45.72) (end 97.79 54.88) (width 0.25) (layer "B.Cu") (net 9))
 (segment (start 56.829 27.619) (end 54.61 25.4) (width 0.25) (layer "B.Cu") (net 9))
 (segment (start 47.371 49.149) (end 45.72 50.8) (width 0.25) (layer "B.Cu") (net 9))
 (segment (start 47.371 35.966) (end 47.092 35.687) (width 0.25) (layer "B.Cu") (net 9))
 (segment (start 46.7276 35.4246) (end 46.7276 31.5856) (width 0.25) (layer "B.Cu") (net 9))
 (segment (start 35.814 53.086) (end 35.814 54.864) (width 0.25) (layer "B.Cu") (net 9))
 (segment (start 97.79 46.99) (end 97.79 25.4) (width 0.25) (layer "B.Cu") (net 9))
 (segment (start 47.371 43.688) (end 48.768 45.085) (width 0.25) (layer "B.Cu") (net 9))
 (segment (start 33.782 56.896) (end 25.527 56.896) (width 0.25) (layer "B.Cu") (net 9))
 (segment (start 72.95 46.7) (end 97.79 46.7) (width 0.25) (layer "B.Cu") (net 9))
 (segment (start 47.371 42.266) (end 47.371 43.688) (width 0.25) (layer "B.Cu") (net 9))
 (segment (start 47.092 35.687) (end 46.99 35.687) (width 0.25) (layer "B.Cu") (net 9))
 (segment (start 97.79 54.88) (end 99.77 56.86) (width 0.25) (layer "B.Cu") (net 9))
 (segment (start 47.371 42.266) (end 47.371 49.149) (width 0.25) (layer "B.Cu") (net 9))
 (segment (start 45.72 50.8) (end 38.1 50.8) (width 0.25) (layer "B.Cu") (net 9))
 (segment (start 46.99 35.687) (end 46.7276 35.4246) (width 0.25) (layer "B.Cu") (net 9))
 (segment (start 97.79 25.4) (end 71.12 25.4) (width 0.25) (layer "B.Cu") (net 9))
 (segment (start 48.26 49.53) (end 48.26 45.72) (width 0.25) (layer "F.Cu") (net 18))
 (segment (start 55.9816 43.18) (end 58.42 43.18) (width 0.25) (layer "F.Cu") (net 18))
 (segment (start 49.3014 44.6786) (end 50.8 44.6786) (width 0.25) (layer "F.Cu") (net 18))
 (segment (start 27.94 53.34) (end 44.45 53.34) (width 0.25) (layer "F.Cu") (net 18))
 (segment (start 44.45 53.34) (end 48.26 49.53) (width 0.25) (layer "F.Cu") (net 18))
 (segment (start 54.483 44.6786) (end 55.9816 43.18) (width 0.25) (layer "F.Cu") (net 18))
 (segment (start 48.26 45.72) (end 49.3014 44.6786) (width 0.25) (layer "F.Cu") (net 18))
 (segment (start 50.8 44.6786) (end 54.483 44.6786) (width 0.25) (layer "F.Cu") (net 18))
 (segment (start 26.67 52.07) (end 27.94 53.34) (width 0.25) (layer "F.Cu") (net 18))
 (segment (start 51.8076 31.5856) (end 51.8076 30.2176) (width 0.25) (layer "F.Cu") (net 11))
 (segment (start 49.53 27.94) (end 49.53 25.4) (width 0.25) (layer "F.Cu") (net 11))
 (segment (start 50.8 49.2286) (end 53.1656 49.2286) (width 0.25) (layer "F.Cu") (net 11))
 (segment (start 58.42 52.07) (end 60.96 52.07) (width 0.25) (layer "F.Cu") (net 11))
 (segment (start 56.007 52.07) (end 58.42 52.07) (width 0.25) (layer "F.Cu") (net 11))
 (segment (start 51.8076 30.2176) (end 49.53 27.94) (width 0.25) (layer "F.Cu") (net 11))
 (segment (start 53.1656 49.2286) (end 56.007 52.07) (width 0.25) (layer "F.Cu") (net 11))
 (via (at 60.96 52.07) (size 0.8) (drill 0.4) (layers "F.Cu" "B.Cu") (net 11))
 (segment (start 53.1756 31.5856) (end 51.8076 31.5856) (width 0.25) (layer "B.Cu") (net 11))
 (segment (start 60.96 39.37) (end 53.1756 31.5856) (width 0.25) (layer "B.Cu") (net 11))
 (segment (start 60.96 52.07) (end 60.96 39.37) (width 0.25) (layer "B.Cu") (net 11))
 (segment (start 56.3118 50.8) (end 58.42 50.8) (width 0.25) (layer "F.Cu") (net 12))
 (segment (start 58.42 50.8) (end 62.23 50.8) (width 0.25) (layer "F.Cu") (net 12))
 (segment (start 54.0904 48.5786) (end 56.3118 50.8) (width 0.25) (layer "F.Cu") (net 12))
 (segment (start 49.2676 31.5856) (end 49.2676 30.2176) (width 0.25) (layer "F.Cu") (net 12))
 (segment (start 50.8 48.5786) (end 54.0904 48.5786) (width 0.25) (layer "F.Cu") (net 12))
 (segment (start 46.99 27.94) (end 46.99 25.4) (width 0.25) (layer "F.Cu") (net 12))
 (segment (start 49.2676 30.2176) (end 46.99 27.94) (width 0.25) (layer "F.Cu") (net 12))
 (via (at 62.23 50.8) (size 0.8) (drill 0.4) (layers "F.Cu" "B.Cu") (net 12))
 (segment (start 62.23 50.8) (end 62.23 29.845) (width 0.25) (layer "B.Cu") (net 12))
 (segment (start 62.23 29.845) (end 51.0082 29.845) (width 0.25) (layer "B.Cu") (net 12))
 (segment (start 51.0082 29.845) (end 49.2676 31.5856) (width 0.25) (layer "B.Cu") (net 12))
 (segment (start 38.1 41.91) (end 37.8714 42.1386) (width 0.25) (layer "F.Cu") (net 2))
 (segment (start 41.0718 41.91) (end 38.1 41.91) (width 0.25) (layer "F.Cu") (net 2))
 (segment (start 43.1904 44.0286) (end 41.0718 41.91) (width 0.25) (layer "F.Cu") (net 2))
 (segment (start 45.075 44.0286) (end 43.1904 44.0286) (width 0.25) (layer "F.Cu") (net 2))
 (segment (start 29.21 54.61) (end 34.29 54.61) (width 0.25) (layer "F.Cu") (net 2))
 (segment (start 38.1 41.91) (end 34.29 41.91) (width 0.25) (layer "F.Cu") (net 2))
 (via (at 34.29 54.61) (size 0.8) (drill 0.4) (layers "F.Cu" "B.Cu") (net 2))
 (via (at 34.29 41.91) (size 0.8) (drill 0.4) (layers "F.Cu" "B.Cu") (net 2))
 (via (at 34.29 41.91) (size 0.8) (drill 0.4) (layers "F.Cu" "B.Cu") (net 2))
 (segment (start 34.29 54.61) (end 34.29 41.91) (width 0.25) (layer "B.Cu") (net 2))
 (segment (start 38.1 43.18) (end 33.02 43.18) (width 0.25) (layer "F.Cu") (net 3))
 (segment (start 40.9702 43.18) (end 38.1 43.18) (width 0.25) (layer "F.Cu") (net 3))
 (segment (start 29.21 52.07) (end 33.02 52.07) (width 0.25) (layer "F.Cu") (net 3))
 (segment (start 45.075 44.6786) (end 42.4688 44.6786) (width 0.25) (layer "F.Cu") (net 3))
 (segment (start 42.4688 44.6786) (end 40.9702 43.18) (width 0.25) (layer "F.Cu") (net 3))
 (via (at 33.02 52.07) (size 0.8) (drill 0.4) (layers "F.Cu" "B.Cu") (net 3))
 (via (at 33.02 43.18) (size 0.8) (drill 0.4) (layers "F.Cu" "B.Cu") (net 3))
 (segment (start 33.02 43.18) (end 33.02 52.07) (width 0.25) (layer "B.Cu") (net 3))
 (segment (start 40.6146 44.45) (end 38.1 44.45) (width 0.25) (layer "F.Cu") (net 4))
 (segment (start 38.1 44.45) (end 29.21 44.45) (width 0.25) (layer "F.Cu") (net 4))
 (segment (start 45.075 45.3286) (end 41.4932 45.3286) (width 0.25) (layer "F.Cu") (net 4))
 (segment (start 41.4932 45.3286) (end 40.6146 44.45) (width 0.25) (layer "F.Cu") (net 4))
 (segment (start 29.21 37.2312) (end 28.7274 36.7486) (width 0.25) (layer "F.Cu") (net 27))
 (segment (start 28.7274 36.7486) (end 28.8088 36.83) (width 0.25) (layer "F.Cu") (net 27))
 (segment (start 28.7274 36.7486) (end 39.5536 36.7486) (width 0.25) (layer "B.Cu") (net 27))
 (segment (start 26.67 44.45) (end 26.67 38.806) (width 0.25) (layer "B.Cu") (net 27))
 (segment (start 39.5536 36.7486) (end 45.071 42.266) (width 0.25) (layer "B.Cu") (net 27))
 (segment (start 26.67 38.806) (end 28.7274 36.7486) (width 0.25) (layer "B.Cu") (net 27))
 (segment (start 55.4078 45.3286) (end 56.2864 44.45) (width 0.25) (layer "F.Cu") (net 17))
 (segment (start 50.8 45.3286) (end 55.4078 45.3286) (width 0.25) (layer "F.Cu") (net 17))
 (segment (start 56.2864 44.45) (end 58.42 44.45) (width 0.25) (layer "F.Cu") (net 17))
 (segment (start 74.64 32.04) (end 80.57 32.04) (width 0.25) (layer "F.Cu") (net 17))
 (segment (start 58.42 44.45) (end 62.23 44.45) (width 0.25) (layer "F.Cu") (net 17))
 (segment (start 62.23 44.45) (end 74.64 32.04) (width 0.25) (layer "F.Cu") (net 17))
 (segment (start 80.3 32.04) (end 80.01 31.75) (width 0.25) (layer "F.Cu") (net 17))
 (segment (start 69.85 49.53) (end 74.93 54.61) (width 0.25) (layer "F.Cu") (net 13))
 (segment (start 54.8374 47.9286) (end 56.4388 49.53) (width 0.25) (layer "F.Cu") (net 13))
 (segment (start 72.39 57.15) (end 74.93 54.61) (width 0.25) (layer "F.Cu") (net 13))
 (segment (start 74.93 54.61) (end 91.02 54.61) (width 0.25) (layer "F.Cu") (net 13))
 (segment (start 71.12 57.15) (end 72.39 57.15) (width 0.25) (layer "F.Cu") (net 13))
 (segment (start 50.8 47.9286) (end 54.8374 47.9286) (width 0.25) (layer "F.Cu") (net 13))
 (segment (start 56.4388 49.53) (end 58.42 49.53) (width 0.25) (layer "F.Cu") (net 13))
 (segment (start 91.02 54.61) (end 93.27 52.36) (width 0.25) (layer "F.Cu") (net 13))
 (segment (start 58.42 49.53) (end 69.85 49.53) (width 0.25) (layer "F.Cu") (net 13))
 (segment (start 84.09 39.37) (end 86.92 42.2) (width 0.25) (layer "F.Cu") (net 16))
 (segment (start 50.8 45.9786) (end 56.231 45.9786) (width 0.25) (layer "F.Cu") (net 16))
 (segment (start 56.4896 45.72) (end 58.42 45.72) (width 0.25) (layer "F.Cu") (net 16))
 (segment (start 64.77 45.72) (end 71.12 39.37) (width 0.25) (layer "F.Cu") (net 16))
 (segment (start 58.42 45.72) (end 64.77 45.72) (width 0.25) (layer "F.Cu") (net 16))
 (segment (start 56.231 45.9786) (end 56.4896 45.72) (width 0.25) (layer "F.Cu") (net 16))
 (segment (start 71.12 39.37) (end 84.09 39.37) (width 0.25) (layer "F.Cu") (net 16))
 (segment (start 50.8 46.6286) (end 56.1282 46.6286) (width 0.25) (layer "F.Cu") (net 15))
 (segment (start 67.31 46.99) (end 72.1 42.2) (width 0.25) (layer "F.Cu") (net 15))
 (segment (start 56.1282 46.6286) (end 56.4896 46.99) (width 0.25) (layer "F.Cu") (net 15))
 (segment (start 58.42 46.99) (end 67.31 46.99) (width 0.25) (layer "F.Cu") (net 15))
 (segment (start 72.1 42.2) (end 72.95 42.2) (width 0.25) (layer "F.Cu") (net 15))
 (segment (start 56.4896 46.99) (end 58.42 46.99) (width 0.25) (layer "F.Cu") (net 15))
 (segment (start 77.76 52.36) (end 80.57 52.36) (width 0.25) (layer "F.Cu") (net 14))
 (segment (start 73.66 48.26) (end 77.76 52.36) (width 0.25) (layer "F.Cu") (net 14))
 (segment (start 58.42 48.26) (end 73.66 48.26) (width 0.25) (layer "F.Cu") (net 14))
 (segment (start 50.8 47.2786) (end 55.6606 47.2786) (width 0.25) (layer "F.Cu") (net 14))
 (segment (start 50.8762 47.2694) (end 50.867 47.2786) (width 0.25) (layer "F.Cu") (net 14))
 (segment (start 50.8 47.2786) (end 50.867 47.2786) (width 0.25) (layer "F.Cu") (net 14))
 (segment (start 56.642 48.26) (end 58.42 48.26) (width 0.25) (layer "F.Cu") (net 14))
 (segment (start 55.6606 47.2786) (end 56.642 48.26) (width 0.25) (layer "F.Cu") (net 14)))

